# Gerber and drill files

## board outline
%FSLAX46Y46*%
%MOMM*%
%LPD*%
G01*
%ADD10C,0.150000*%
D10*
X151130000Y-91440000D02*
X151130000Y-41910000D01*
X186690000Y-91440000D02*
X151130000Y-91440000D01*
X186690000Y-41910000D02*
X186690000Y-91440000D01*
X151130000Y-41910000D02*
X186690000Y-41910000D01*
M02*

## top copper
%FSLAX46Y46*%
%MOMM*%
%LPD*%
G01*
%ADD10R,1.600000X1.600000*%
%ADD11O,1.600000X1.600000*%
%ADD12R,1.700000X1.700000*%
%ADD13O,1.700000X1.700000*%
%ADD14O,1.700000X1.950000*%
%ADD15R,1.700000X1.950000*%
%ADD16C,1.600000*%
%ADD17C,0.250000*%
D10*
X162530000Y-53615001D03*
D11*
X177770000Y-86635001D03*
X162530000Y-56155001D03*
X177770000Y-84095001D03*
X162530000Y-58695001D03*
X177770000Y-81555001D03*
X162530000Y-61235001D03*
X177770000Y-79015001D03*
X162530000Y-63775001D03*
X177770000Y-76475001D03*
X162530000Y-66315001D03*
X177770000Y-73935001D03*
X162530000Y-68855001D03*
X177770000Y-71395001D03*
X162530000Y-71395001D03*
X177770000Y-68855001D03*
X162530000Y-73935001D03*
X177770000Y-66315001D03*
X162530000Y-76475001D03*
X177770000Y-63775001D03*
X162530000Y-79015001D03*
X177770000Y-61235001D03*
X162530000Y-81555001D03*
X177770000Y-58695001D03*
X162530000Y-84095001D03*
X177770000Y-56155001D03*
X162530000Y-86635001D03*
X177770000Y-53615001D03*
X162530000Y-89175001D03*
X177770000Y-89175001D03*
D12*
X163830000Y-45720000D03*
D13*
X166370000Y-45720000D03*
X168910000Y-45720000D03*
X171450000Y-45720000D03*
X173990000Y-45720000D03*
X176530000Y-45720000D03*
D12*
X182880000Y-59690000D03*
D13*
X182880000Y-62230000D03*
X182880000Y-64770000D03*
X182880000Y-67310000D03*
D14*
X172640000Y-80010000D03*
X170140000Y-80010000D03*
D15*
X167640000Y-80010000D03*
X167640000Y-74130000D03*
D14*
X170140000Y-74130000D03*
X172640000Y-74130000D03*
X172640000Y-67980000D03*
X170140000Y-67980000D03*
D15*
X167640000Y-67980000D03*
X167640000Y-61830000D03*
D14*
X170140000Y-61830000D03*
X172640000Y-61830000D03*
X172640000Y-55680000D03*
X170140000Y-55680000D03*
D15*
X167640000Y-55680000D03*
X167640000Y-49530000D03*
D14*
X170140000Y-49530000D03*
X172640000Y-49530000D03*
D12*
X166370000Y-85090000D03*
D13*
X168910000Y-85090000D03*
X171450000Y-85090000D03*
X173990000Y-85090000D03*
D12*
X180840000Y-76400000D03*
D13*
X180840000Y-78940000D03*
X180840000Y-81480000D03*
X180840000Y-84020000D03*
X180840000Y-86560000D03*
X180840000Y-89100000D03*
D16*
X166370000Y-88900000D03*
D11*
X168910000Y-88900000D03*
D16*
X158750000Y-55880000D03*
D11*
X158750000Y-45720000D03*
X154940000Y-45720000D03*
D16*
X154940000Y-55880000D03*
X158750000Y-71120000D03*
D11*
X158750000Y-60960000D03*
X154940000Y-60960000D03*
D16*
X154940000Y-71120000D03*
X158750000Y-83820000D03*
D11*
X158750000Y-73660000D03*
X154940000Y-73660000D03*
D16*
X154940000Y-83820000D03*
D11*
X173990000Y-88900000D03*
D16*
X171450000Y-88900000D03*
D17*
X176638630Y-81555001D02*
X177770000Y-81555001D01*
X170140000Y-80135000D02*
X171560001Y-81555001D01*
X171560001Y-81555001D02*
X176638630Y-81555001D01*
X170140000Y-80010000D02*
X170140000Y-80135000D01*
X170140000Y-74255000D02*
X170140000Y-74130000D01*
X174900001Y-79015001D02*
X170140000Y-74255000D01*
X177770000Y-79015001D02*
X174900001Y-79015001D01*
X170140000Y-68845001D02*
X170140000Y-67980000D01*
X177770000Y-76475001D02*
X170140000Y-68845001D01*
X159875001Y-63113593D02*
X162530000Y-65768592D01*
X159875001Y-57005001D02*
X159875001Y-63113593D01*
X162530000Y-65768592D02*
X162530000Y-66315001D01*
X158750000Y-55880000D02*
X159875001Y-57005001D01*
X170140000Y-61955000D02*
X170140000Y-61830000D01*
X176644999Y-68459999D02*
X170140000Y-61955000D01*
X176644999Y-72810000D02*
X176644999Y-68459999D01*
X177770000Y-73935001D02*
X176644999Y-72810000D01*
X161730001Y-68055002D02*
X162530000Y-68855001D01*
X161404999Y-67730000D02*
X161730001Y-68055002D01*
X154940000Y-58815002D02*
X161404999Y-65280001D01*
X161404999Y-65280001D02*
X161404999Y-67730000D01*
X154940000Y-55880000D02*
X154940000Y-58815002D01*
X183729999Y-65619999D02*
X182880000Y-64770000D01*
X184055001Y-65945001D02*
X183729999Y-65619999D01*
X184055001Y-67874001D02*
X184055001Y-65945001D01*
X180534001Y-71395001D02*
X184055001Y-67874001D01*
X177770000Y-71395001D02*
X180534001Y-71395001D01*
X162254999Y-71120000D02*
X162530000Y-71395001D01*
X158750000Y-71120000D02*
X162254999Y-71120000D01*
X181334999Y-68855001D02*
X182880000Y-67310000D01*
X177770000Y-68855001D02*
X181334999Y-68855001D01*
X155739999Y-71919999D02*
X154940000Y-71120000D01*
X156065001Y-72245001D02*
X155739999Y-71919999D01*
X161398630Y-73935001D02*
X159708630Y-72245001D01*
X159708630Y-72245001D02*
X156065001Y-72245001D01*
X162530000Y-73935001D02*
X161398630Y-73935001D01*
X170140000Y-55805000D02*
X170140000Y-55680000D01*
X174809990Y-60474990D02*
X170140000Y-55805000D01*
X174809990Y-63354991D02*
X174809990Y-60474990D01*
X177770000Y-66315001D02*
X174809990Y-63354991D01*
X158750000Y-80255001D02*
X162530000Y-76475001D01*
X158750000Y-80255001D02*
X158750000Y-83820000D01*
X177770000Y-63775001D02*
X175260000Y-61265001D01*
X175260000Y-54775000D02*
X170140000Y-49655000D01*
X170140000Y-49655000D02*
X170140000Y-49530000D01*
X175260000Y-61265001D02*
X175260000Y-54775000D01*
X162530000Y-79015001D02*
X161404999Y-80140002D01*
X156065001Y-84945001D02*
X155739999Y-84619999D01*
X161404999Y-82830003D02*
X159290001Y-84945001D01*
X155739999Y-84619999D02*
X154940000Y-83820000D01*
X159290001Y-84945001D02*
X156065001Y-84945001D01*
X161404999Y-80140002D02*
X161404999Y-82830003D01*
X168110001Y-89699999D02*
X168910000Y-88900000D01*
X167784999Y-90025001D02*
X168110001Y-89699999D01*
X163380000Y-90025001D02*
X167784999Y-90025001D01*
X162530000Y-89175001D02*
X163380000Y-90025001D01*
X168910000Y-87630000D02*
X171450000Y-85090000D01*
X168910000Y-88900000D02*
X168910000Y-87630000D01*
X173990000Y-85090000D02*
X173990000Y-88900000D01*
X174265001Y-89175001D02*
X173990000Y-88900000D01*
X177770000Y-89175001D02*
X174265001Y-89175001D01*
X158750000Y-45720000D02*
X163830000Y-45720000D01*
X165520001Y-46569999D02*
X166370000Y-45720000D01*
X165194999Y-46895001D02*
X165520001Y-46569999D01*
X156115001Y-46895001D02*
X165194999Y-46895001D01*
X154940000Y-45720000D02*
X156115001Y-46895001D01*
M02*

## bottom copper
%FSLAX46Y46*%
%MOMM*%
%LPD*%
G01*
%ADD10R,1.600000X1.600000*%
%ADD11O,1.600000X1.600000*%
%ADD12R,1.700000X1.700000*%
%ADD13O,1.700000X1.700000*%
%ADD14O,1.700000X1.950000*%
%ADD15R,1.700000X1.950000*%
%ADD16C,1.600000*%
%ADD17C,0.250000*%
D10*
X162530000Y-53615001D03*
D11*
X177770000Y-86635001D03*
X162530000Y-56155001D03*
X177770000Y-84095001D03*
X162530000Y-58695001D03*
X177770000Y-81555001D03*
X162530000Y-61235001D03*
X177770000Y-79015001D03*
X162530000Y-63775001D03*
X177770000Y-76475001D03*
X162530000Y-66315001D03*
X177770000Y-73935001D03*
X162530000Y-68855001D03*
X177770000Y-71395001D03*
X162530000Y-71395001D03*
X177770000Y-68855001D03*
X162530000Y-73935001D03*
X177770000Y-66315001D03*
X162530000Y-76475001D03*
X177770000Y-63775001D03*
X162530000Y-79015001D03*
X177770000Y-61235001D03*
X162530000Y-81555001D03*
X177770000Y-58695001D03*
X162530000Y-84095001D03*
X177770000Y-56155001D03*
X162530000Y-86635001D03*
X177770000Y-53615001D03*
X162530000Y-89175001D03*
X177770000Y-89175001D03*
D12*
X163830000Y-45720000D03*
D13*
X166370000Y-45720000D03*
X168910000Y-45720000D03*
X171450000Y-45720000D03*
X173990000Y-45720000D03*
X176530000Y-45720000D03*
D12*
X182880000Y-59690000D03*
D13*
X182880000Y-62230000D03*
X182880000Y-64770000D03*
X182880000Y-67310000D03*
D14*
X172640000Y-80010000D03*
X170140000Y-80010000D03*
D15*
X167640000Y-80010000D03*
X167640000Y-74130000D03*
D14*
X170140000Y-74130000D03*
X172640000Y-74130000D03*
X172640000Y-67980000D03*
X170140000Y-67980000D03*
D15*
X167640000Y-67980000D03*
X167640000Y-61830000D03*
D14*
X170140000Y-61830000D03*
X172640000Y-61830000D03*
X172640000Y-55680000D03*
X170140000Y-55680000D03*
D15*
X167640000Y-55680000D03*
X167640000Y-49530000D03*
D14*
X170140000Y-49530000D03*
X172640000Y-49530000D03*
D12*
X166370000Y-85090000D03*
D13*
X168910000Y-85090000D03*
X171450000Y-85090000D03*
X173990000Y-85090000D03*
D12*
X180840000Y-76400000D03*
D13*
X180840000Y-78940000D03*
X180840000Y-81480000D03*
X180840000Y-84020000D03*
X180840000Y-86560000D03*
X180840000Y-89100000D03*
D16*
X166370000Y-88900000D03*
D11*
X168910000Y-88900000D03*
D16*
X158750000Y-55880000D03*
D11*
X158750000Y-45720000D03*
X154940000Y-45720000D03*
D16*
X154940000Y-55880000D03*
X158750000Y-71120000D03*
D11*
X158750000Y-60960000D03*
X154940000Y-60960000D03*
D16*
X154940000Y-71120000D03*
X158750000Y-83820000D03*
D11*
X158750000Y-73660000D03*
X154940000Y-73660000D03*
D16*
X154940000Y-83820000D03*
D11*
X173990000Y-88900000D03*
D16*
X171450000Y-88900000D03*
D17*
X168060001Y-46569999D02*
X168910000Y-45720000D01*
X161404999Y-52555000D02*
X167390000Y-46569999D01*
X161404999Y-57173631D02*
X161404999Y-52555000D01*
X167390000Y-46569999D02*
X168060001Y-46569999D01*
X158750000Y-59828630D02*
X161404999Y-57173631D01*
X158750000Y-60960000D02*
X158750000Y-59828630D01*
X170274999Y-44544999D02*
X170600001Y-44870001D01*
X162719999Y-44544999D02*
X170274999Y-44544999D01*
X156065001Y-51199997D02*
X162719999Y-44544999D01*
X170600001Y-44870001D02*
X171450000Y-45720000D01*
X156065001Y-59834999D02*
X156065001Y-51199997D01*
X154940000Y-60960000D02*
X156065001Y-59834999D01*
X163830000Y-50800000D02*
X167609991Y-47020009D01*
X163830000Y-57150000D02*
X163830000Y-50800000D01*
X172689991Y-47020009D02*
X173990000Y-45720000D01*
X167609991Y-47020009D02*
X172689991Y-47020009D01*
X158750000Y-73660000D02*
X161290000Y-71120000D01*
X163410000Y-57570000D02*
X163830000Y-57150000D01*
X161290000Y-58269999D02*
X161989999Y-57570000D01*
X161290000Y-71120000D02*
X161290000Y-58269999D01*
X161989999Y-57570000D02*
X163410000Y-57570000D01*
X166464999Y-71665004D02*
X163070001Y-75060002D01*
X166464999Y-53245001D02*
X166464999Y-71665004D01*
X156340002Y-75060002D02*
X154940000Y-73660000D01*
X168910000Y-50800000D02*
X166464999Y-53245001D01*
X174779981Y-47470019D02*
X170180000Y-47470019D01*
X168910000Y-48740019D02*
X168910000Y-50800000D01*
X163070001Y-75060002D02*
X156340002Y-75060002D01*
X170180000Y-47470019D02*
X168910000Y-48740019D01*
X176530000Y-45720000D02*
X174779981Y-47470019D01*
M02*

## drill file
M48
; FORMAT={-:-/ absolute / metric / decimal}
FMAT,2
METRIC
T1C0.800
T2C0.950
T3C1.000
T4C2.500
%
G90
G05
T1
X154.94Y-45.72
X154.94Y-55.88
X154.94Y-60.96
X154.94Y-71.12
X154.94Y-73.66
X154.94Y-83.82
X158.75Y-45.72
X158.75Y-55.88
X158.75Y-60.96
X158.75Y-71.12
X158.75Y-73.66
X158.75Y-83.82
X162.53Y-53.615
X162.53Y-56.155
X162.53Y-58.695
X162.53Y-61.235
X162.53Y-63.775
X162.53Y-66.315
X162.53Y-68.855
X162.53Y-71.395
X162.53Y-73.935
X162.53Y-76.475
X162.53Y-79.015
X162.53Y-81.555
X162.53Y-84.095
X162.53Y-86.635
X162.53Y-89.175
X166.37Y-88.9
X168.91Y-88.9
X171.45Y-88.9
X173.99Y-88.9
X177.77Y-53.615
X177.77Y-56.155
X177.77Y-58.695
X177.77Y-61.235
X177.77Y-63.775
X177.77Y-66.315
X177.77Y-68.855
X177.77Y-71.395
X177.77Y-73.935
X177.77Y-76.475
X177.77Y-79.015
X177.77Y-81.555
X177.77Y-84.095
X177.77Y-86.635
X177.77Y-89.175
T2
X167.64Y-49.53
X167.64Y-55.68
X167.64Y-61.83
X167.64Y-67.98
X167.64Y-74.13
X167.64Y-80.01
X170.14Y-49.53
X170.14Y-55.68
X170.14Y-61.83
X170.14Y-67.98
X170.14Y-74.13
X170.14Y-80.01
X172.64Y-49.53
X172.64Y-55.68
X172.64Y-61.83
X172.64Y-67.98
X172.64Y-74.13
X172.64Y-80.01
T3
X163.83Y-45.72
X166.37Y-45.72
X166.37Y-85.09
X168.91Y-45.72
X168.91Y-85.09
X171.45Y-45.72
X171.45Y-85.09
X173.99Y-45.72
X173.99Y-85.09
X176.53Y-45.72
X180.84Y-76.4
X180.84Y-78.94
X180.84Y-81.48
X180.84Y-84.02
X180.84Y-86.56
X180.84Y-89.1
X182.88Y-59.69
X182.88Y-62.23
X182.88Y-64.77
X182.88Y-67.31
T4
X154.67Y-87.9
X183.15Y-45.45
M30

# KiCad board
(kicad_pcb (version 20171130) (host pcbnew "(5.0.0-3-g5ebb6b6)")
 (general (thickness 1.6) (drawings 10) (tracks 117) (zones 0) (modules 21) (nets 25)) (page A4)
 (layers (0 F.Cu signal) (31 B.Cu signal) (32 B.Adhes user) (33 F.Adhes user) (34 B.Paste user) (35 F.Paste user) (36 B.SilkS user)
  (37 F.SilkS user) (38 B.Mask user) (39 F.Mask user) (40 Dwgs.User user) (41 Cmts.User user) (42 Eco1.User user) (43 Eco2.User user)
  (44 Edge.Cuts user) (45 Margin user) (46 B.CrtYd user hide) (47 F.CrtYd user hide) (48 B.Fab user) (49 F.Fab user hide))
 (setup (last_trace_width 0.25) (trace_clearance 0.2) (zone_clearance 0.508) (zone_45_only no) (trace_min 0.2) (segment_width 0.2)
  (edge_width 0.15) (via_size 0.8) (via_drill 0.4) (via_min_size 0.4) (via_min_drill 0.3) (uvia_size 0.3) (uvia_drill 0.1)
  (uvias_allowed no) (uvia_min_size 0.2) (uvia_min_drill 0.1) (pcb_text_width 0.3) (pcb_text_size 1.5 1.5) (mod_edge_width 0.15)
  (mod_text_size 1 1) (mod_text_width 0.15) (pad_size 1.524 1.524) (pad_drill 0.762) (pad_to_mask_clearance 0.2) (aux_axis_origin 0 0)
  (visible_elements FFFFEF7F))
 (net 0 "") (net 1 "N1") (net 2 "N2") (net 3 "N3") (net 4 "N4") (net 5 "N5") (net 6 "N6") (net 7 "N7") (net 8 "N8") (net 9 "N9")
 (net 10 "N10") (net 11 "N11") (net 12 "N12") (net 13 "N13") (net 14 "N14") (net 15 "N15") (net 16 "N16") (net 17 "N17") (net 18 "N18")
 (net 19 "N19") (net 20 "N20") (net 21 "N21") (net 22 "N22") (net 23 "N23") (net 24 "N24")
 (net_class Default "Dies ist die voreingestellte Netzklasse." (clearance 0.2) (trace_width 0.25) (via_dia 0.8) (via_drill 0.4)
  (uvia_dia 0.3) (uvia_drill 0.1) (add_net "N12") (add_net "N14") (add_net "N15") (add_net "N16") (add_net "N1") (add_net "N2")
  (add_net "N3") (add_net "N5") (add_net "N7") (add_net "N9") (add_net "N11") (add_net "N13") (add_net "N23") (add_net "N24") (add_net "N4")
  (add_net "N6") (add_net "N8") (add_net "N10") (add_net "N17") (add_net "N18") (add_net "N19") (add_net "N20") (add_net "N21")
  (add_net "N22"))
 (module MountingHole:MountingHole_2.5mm (layer F.Cu) (at 154.67 87.9)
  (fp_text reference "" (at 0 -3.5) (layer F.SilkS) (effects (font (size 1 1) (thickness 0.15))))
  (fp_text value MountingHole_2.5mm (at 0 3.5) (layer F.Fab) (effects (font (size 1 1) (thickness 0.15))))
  (pad 1 np_thru_hole circle (at 0 0) (size 2.5 2.5) (drill 2.5) (layers *.Cu *.Mask)))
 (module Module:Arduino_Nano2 (layer F.Cu) (at 162.53 53.615001)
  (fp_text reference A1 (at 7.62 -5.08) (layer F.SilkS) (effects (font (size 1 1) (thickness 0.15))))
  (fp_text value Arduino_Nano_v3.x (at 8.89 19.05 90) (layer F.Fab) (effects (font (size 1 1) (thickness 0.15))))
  (pad 1 thru_hole rect (at 0 0) (size 1.6 1.6) (drill 0.8) (layers *.Cu *.Mask))
  (pad 17 thru_hole oval (at 15.24 33.02) (size 1.6 1.6) (drill 0.8) (layers *.Cu *.Mask))
  (pad 2 thru_hole oval (at 0 2.54) (size 1.6 1.6) (drill 0.8) (layers *.Cu *.Mask))
  (pad 18 thru_hole oval (at 15.24 30.48) (size 1.6 1.6) (drill 0.8) (layers *.Cu *.Mask))
  (pad 3 thru_hole oval (at 0 5.08) (size 1.6 1.6) (drill 0.8) (layers *.Cu *.Mask))
  (pad 19 thru_hole oval (at 15.24 27.94) (size 1.6 1.6) (drill 0.8) (layers *.Cu *.Mask) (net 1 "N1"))
  (pad 4 thru_hole oval (at 0 7.62) (size 1.6 1.6) (drill 0.8) (layers *.Cu *.Mask))
  (pad 20 thru_hole oval (at 15.24 25.4) (size 1.6 1.6) (drill 0.8) (layers *.Cu *.Mask) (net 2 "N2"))
  (pad 5 thru_hole oval (at 0 10.16) (size 1.6 1.6) (drill 0.8) (layers *.Cu *.Mask))
  (pad 21 thru_hole oval (at 15.24 22.86) (size 1.6 1.6) (drill 0.8) (layers *.Cu *.Mask) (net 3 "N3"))
  (pad 6 thru_hole oval (at 0 12.7) (size 1.6 1.6) (drill 0.8) (layers *.Cu *.Mask) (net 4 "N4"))
  (pad 22 thru_hole oval (at 15.24 20.32) (size 1.6 1.6) (drill 0.8) (layers *.Cu *.Mask) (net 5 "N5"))
  (pad 7 thru_hole oval (at 0 15.24) (size 1.6 1.6) (drill 0.8) (layers *.Cu *.Mask) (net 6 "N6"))
  (pad 23 thru_hole oval (at 15.24 17.78) (size 1.6 1.6) (drill 0.8) (layers *.Cu *.Mask) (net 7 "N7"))
  (pad 8 thru_hole oval (at 0 17.78) (size 1.6 1.6) (drill 0.8) (layers *.Cu *.Mask) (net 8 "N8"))
  (pad 24 thru_hole oval (at 15.24 15.24) (size 1.6 1.6) (drill 0.8) (layers *.Cu *.Mask) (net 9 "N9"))
  (pad 9 thru_hole oval (at 0 20.32) (size 1.6 1.6) (drill 0.8) (layers *.Cu *.Mask) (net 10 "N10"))
  (pad 25 thru_hole oval (at 15.24 12.7) (size 1.6 1.6) (drill 0.8) (layers *.Cu *.Mask) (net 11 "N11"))
  (pad 10 thru_hole oval (at 0 22.86) (size 1.6 1.6) (drill 0.8) (layers *.Cu *.Mask) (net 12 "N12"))
  (pad 26 thru_hole oval (at 15.24 10.16) (size 1.6 1.6) (drill 0.8) (layers *.Cu *.Mask) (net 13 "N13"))
  (pad 11 thru_hole oval (at 0 25.4) (size 1.6 1.6) (drill 0.8) (layers *.Cu *.Mask) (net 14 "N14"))
  (pad 27 thru_hole oval (at 15.24 7.62) (size 1.6 1.6) (drill 0.8) (layers *.Cu *.Mask))
  (pad 12 thru_hole oval (at 0 27.94) (size 1.6 1.6) (drill 0.8) (layers *.Cu *.Mask))
  (pad 28 thru_hole oval (at 15.24 5.08) (size 1.6 1.6) (drill 0.8) (layers *.Cu *.Mask))
  (pad 13 thru_hole oval (at 0 30.48) (size 1.6 1.6) (drill 0.8) (layers *.Cu *.Mask))
  (pad 29 thru_hole oval (at 15.24 2.54) (size 1.6 1.6) (drill 0.8) (layers *.Cu *.Mask))
  (pad 14 thru_hole oval (at 0 33.02) (size 1.6 1.6) (drill 0.8) (layers *.Cu *.Mask))
  (pad 30 thru_hole oval (at 15.24 0) (size 1.6 1.6) (drill 0.8) (layers *.Cu *.Mask))
  (pad 15 thru_hole oval (at 0 35.56) (size 1.6 1.6) (drill 0.8) (layers *.Cu *.Mask) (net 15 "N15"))
  (pad 16 thru_hole oval (at 15.24 35.56) (size 1.6 1.6) (drill 0.8) (layers *.Cu *.Mask) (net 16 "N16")))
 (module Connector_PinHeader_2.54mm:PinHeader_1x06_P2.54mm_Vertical (layer F.Cu) (at 163.83 45.72 90)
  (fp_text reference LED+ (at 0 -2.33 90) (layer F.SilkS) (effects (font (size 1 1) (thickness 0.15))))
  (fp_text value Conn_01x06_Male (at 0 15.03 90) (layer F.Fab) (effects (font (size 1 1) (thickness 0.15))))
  (pad 1 thru_hole rect (at 0 0 90) (size 1.7 1.7) (drill 1) (layers *.Cu *.Mask) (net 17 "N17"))
  (pad 2 thru_hole oval (at 0 2.54 90) (size 1.7 1.7) (drill 1) (layers *.Cu *.Mask) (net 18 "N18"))
  (pad 3 thru_hole oval (at 0 5.08 90) (size 1.7 1.7) (drill 1) (layers *.Cu *.Mask) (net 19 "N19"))
  (pad 4 thru_hole oval (at 0 7.62 90) (size 1.7 1.7) (drill 1) (layers *.Cu *.Mask) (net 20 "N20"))
  (pad 5 thru_hole oval (at 0 10.16 90) (size 1.7 1.7) (drill 1) (layers *.Cu *.Mask) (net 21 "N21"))
  (pad 6 thru_hole oval (at 0 12.7 90) (size 1.7 1.7) (drill 1) (layers *.Cu *.Mask) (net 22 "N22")))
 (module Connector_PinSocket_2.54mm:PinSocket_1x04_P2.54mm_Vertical (layer F.Cu) (at 182.88 59.69)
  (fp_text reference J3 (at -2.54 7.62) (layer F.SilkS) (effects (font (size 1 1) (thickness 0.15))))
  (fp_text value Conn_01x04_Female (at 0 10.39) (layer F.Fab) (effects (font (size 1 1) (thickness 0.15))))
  (pad 1 thru_hole rect (at 0 0) (size 1.7 1.7) (drill 1) (layers *.Cu *.Mask))
  (pad 2 thru_hole oval (at 0 2.54) (size 1.7 1.7) (drill 1) (layers *.Cu *.Mask))
  (pad 3 thru_hole oval (at 0 5.08) (size 1.7 1.7) (drill 1) (layers *.Cu *.Mask) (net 7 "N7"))
  (pad 4 thru_hole oval (at 0 7.62) (size 1.7 1.7) (drill 1) (layers *.Cu *.Mask) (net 9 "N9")))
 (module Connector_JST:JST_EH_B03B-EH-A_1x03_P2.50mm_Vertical (layer F.Cu) (at 167.64 80.01)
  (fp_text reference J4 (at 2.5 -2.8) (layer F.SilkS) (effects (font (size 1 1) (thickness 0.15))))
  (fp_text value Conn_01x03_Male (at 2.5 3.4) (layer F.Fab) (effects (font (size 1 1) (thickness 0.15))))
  (pad 3 thru_hole oval (at 5 0) (size 1.7 1.95) (drill 0.95) (layers *.Cu *.Mask))
  (pad 2 thru_hole oval (at 2.5 0) (size 1.7 1.95) (drill 0.95) (layers *.Cu *.Mask) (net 1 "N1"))
  (pad 1 thru_hole rect (at 0 0) (size 1.7 1.95) (drill 0.95) (layers *.Cu *.Mask)))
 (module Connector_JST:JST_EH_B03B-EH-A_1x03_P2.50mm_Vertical (layer F.Cu) (at 167.64 74.13)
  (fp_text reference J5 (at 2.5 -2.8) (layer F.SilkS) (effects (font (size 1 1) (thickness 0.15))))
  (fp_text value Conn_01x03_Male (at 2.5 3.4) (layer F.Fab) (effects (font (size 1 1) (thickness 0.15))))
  (pad 1 thru_hole rect (at 0 0) (size 1.7 1.95) (drill 0.95) (layers *.Cu *.Mask))
  (pad 2 thru_hole oval (at 2.5 0) (size 1.7 1.95) (drill 0.95) (layers *.Cu *.Mask) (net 2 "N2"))
  (pad 3 thru_hole oval (at 5 0) (size 1.7 1.95) (drill 0.95) (layers *.Cu *.Mask)))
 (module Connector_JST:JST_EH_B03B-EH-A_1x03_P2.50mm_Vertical (layer F.Cu) (at 167.64 67.98)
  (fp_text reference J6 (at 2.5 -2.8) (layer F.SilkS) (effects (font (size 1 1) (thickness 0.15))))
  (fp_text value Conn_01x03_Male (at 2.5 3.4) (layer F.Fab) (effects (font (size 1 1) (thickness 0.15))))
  (pad 3 thru_hole oval (at 5 0) (size 1.7 1.95) (drill 0.95) (layers *.Cu *.Mask))
  (pad 2 thru_hole oval (at 2.5 0) (size 1.7 1.95) (drill 0.95) (layers *.Cu *.Mask) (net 3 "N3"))
  (pad 1 thru_hole rect (at 0 0) (size 1.7 1.95) (drill 0.95) (layers *.Cu *.Mask)))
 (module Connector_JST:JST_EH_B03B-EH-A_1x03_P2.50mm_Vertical (layer F.Cu) (at 167.64 61.83)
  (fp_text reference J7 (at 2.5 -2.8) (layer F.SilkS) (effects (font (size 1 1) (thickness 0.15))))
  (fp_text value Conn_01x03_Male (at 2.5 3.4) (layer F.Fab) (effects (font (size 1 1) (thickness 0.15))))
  (pad 1 thru_hole rect (at 0 0) (size 1.7 1.95) (drill 0.95) (layers *.Cu *.Mask))
  (pad 2 thru_hole oval (at 2.5 0) (size 1.7 1.95) (drill 0.95) (layers *.Cu *.Mask) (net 5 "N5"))
  (pad 3 thru_hole oval (at 5 0) (size 1.7 1.95) (drill 0.95) (layers *.Cu *.Mask)))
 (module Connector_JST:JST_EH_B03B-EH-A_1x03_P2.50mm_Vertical (layer F.Cu) (at 167.64 55.68)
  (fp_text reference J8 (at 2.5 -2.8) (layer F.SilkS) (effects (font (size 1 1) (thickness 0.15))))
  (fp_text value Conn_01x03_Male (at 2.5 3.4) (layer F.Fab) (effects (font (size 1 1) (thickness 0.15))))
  (pad 3 thru_hole oval (at 5 0) (size 1.7 1.95) (drill 0.95) (layers *.Cu *.Mask))
  (pad 2 thru_hole oval (at 2.5 0) (size 1.7 1.95) (drill 0.95) (layers *.Cu *.Mask) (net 11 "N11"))
  (pad 1 thru_hole rect (at 0 0) (size 1.7 1.95) (drill 0.95) (layers *.Cu *.Mask)))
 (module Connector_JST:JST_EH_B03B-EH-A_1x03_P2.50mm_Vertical (layer F.Cu) (at 167.64 49.53)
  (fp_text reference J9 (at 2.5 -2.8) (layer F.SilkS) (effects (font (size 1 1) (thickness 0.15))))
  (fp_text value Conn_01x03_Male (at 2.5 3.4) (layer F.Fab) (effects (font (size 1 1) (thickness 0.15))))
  (pad 1 thru_hole rect (at 0 0) (size 1.7 1.95) (drill 0.95) (layers *.Cu *.Mask))
  (pad 2 thru_hole oval (at 2.5 0) (size 1.7 1.95) (drill 0.95) (layers *.Cu *.Mask) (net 13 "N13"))
  (pad 3 thru_hole oval (at 5 0) (size 1.7 1.95) (drill 0.95) (layers *.Cu *.Mask)))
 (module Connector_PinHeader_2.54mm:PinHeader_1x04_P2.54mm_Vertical (layer F.Cu) (at 166.37 85.09 90)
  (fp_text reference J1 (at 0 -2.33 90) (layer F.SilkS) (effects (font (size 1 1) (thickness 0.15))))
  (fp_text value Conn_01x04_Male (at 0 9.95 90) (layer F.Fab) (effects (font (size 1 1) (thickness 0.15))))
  (pad 1 thru_hole rect (at 0 0 90) (size 1.7 1.7) (drill 1) (layers *.Cu *.Mask))
  (pad 2 thru_hole oval (at 0 2.54 90) (size 1.7 1.7) (drill 1) (layers *.Cu *.Mask))
  (pad 3 thru_hole oval (at 0 5.08 90) (size 1.7 1.7) (drill 1) (layers *.Cu *.Mask) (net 15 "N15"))
  (pad 4 thru_hole oval (at 0 7.62 90) (size 1.7 1.7) (drill 1) (layers *.Cu *.Mask) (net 16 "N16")))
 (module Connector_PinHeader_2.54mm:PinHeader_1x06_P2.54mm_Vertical (layer F.Cu) (at 180.84 76.4)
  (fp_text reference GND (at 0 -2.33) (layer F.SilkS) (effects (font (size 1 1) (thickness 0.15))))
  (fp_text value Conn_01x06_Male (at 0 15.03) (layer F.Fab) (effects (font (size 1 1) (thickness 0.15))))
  (pad 1 thru_hole rect (at 0 0) (size 1.7 1.7) (drill 1) (layers *.Cu *.Mask))
  (pad 2 thru_hole oval (at 0 2.54) (size 1.7 1.7) (drill 1) (layers *.Cu *.Mask))
  (pad 3 thru_hole oval (at 0 5.08) (size 1.7 1.7) (drill 1) (layers *.Cu *.Mask))
  (pad 4 thru_hole oval (at 0 7.62) (size 1.7 1.7) (drill 1) (layers *.Cu *.Mask))
  (pad 5 thru_hole oval (at 0 10.16) (size 1.7 1.7) (drill 1) (layers *.Cu *.Mask))
  (pad 6 thru_hole oval (at 0 12.7) (size 1.7 1.7) (drill 1) (layers *.Cu *.Mask)))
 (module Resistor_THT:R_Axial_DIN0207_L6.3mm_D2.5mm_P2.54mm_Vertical (layer F.Cu) (at 166.37 88.9)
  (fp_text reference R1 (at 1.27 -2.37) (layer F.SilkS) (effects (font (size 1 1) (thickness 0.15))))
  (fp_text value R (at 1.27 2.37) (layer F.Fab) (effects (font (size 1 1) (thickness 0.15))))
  (pad 1 thru_hole circle (at 0 0) (size 1.6 1.6) (drill 0.8) (layers *.Cu *.Mask))
  (pad 2 thru_hole oval (at 2.54 0) (size 1.6 1.6) (drill 0.8) (layers *.Cu *.Mask) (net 15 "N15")))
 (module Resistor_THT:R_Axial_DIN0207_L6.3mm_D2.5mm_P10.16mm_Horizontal (layer F.Cu) (at 158.75 55.88 90)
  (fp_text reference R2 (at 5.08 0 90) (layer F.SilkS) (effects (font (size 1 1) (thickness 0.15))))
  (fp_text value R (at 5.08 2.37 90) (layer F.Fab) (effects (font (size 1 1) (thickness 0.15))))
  (pad 1 thru_hole circle (at 0 0 90) (size 1.6 1.6) (drill 0.8) (layers *.Cu *.Mask) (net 4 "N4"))
  (pad 2 thru_hole oval (at 10.16 0 90) (size 1.6 1.6) (drill 0.8) (layers *.Cu *.Mask) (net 17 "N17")))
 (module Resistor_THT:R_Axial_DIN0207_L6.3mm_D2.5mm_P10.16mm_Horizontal (layer F.Cu) (at 154.94 55.88 90)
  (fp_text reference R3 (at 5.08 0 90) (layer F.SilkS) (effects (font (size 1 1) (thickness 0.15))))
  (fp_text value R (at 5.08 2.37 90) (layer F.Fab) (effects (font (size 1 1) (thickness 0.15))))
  (pad 2 thru_hole oval (at 10.16 0 90) (size 1.6 1.6) (drill 0.8) (layers *.Cu *.Mask) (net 18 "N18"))
  (pad 1 thru_hole circle (at 0 0 90) (size 1.6 1.6) (drill 0.8) (layers *.Cu *.Mask) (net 6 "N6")))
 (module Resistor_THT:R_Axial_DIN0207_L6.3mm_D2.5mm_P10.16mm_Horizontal (layer F.Cu) (at 158.75 71.12 90)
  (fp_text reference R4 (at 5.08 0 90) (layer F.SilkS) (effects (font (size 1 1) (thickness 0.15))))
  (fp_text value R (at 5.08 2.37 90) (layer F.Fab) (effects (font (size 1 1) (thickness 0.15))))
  (pad 1 thru_hole circle (at 0 0 90) (size 1.6 1.6) (drill 0.8) (layers *.Cu *.Mask) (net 8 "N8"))
  (pad 2 thru_hole oval (at 10.16 0 90) (size 1.6 1.6) (drill 0.8) (layers *.Cu *.Mask) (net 19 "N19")))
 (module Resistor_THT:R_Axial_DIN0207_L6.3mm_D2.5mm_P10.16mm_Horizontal (layer F.Cu) (at 154.94 71.12 90)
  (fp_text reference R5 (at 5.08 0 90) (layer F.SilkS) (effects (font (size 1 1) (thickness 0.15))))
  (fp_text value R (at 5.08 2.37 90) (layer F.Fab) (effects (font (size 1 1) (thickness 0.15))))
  (pad 2 thru_hole oval (at 10.16 0 90) (size 1.6 1.6) (drill 0.8) (layers *.Cu *.Mask) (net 20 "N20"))
  (pad 1 thru_hole circle (at 0 0 90) (size 1.6 1.6) (drill 0.8) (layers *.Cu *.Mask) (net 10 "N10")))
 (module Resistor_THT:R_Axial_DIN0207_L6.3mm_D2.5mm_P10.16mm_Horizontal (layer F.Cu) (at 158.75 83.82 90)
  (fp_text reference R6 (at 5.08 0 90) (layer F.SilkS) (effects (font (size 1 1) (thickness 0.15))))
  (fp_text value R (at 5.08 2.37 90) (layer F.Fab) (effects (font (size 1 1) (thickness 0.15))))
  (pad 1 thru_hole circle (at 0 0 90) (size 1.6 1.6) (drill 0.8) (layers *.Cu *.Mask) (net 12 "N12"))
  (pad 2 thru_hole oval (at 10.16 0 90) (size 1.6 1.6) (drill 0.8) (layers *.Cu *.Mask) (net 21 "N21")))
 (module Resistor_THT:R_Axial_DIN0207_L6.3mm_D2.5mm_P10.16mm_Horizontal (layer F.Cu) (at 154.94 83.82 90)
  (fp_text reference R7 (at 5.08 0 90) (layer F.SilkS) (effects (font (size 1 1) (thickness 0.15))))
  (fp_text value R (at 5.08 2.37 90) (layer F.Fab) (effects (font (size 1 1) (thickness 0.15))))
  (pad 2 thru_hole oval (at 10.16 0 90) (size 1.6 1.6) (drill 0.8) (layers *.Cu *.Mask) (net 22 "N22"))
  (pad 1 thru_hole circle (at 0 0 90) (size 1.6 1.6) (drill 0.8) (layers *.Cu *.Mask) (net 14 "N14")))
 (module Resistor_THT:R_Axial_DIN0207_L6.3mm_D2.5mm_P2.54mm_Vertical (layer F.Cu) (at 171.45 88.9)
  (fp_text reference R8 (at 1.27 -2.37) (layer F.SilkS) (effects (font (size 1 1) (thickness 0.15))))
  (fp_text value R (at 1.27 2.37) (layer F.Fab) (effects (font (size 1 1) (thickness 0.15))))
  (pad 2 thru_hole oval (at 2.54 0) (size 1.6 1.6) (drill 0.8) (layers *.Cu *.Mask) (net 16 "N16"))
  (pad 1 thru_hole circle (at 0 0) (size 1.6 1.6) (drill 0.8) (layers *.Cu *.Mask)))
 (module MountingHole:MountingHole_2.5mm (layer F.Cu) (at 183.15 45.45)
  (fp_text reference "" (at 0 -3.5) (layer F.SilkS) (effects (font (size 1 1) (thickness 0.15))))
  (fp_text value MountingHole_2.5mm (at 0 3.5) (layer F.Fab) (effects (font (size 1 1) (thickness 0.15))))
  (pad 1 np_thru_hole circle (at 0 0) (size 2.5 2.5) (drill 2.5) (layers *.Cu *.Mask)))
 (gr_line (start 151.13 91.44) (end 151.13 41.91) (layer Edge.Cuts) (width 0.15))
 (gr_line (start 186.69 91.44) (end 151.13 91.44) (layer Edge.Cuts) (width 0.15))
 (gr_line (start 186.69 41.91) (end 186.69 91.44) (layer Edge.Cuts) (width 0.15))
 (gr_line (start 151.13 41.91) (end 186.69 41.91) (layer Edge.Cuts) (width 0.15))
 (segment (start 176.63863 81.555001) (end 177.77 81.555001) (width 0.25) (layer F.Cu) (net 1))
 (segment (start 170.14 80.135) (end 171.560001 81.555001) (width 0.25) (layer F.Cu) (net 1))
 (segment (start 171.560001 81.555001) (end 176.63863 81.555001) (width 0.25) (layer F.Cu) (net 1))
 (segment (start 170.14 80.01) (end 170.14 80.135) (width 0.25) (layer F.Cu) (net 1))
 (segment (start 170.14 74.255) (end 170.14 74.13) (width 0.25) (layer F.Cu) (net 2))
 (segment (start 174.900001 79.015001) (end 170.14 74.255) (width 0.25) (layer F.Cu) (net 2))
 (segment (start 177.77 79.015001) (end 174.900001 79.015001) (width 0.25) (layer F.Cu) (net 2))
 (segment (start 170.14 68.845001) (end 170.14 67.98) (width 0.25) (layer F.Cu) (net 3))
 (segment (start 177.77 76.475001) (end 170.14 68.845001) (width 0.25) (layer F.Cu) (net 3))
 (segment (start 159.875001 63.113593) (end 162.53 65.768592) (width 0.25) (layer F.Cu) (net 4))
 (segment (start 159.875001 57.005001) (end 159.875001 63.113593) (width 0.25) (layer F.Cu) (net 4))
 (segment (start 162.53 65.768592) (end 162.53 66.315001) (width 0.25) (layer F.Cu) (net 4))
 (segment (start 158.75 55.88) (end 159.875001 57.005001) (width 0.25) (layer F.Cu) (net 4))
 (segment (start 170.14 61.955) (end 170.14 61.83) (width 0.25) (layer F.Cu) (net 5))
 (segment (start 176.644999 68.459999) (end 170.14 61.955) (width 0.25) (layer F.Cu) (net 5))
 (segment (start 176.644999 72.81) (end 176.644999 68.459999) (width 0.25) (layer F.Cu) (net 5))
 (segment (start 177.77 73.935001) (end 176.644999 72.81) (width 0.25) (layer F.Cu) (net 5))
 (segment (start 161.730001 68.055002) (end 162.53 68.855001) (width 0.25) (layer F.Cu) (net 6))
 (segment (start 161.404999 67.73) (end 161.730001 68.055002) (width 0.25) (layer F.Cu) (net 6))
 (segment (start 154.94 58.815002) (end 161.404999 65.280001) (width 0.25) (layer F.Cu) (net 6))
 (segment (start 161.404999 65.280001) (end 161.404999 67.73) (width 0.25) (layer F.Cu) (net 6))
 (segment (start 154.94 55.88) (end 154.94 58.815002) (width 0.25) (layer F.Cu) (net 6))
 (segment (start 183.729999 65.619999) (end 182.88 64.77) (width 0.25) (layer F.Cu) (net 7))
 (segment (start 184.055001 65.945001) (end 183.729999 65.619999) (width 0.25) (layer F.Cu) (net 7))
 (segment (start 184.055001 67.874001) (end 184.055001 65.945001) (width 0.25) (layer F.Cu) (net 7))
 (segment (start 180.534001 71.395001) (end 184.055001 67.874001) (width 0.25) (layer F.Cu) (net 7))
 (segment (start 177.77 71.395001) (end 180.534001 71.395001) (width 0.25) (layer F.Cu) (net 7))
 (segment (start 162.254999 71.12) (end 162.53 71.395001) (width 0.25) (layer F.Cu) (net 8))
 (segment (start 158.75 71.12) (end 162.254999 71.12) (width 0.25) (layer F.Cu) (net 8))
 (segment (start 181.334999 68.855001) (end 182.88 67.31) (width 0.25) (layer F.Cu) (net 9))
 (segment (start 177.77 68.855001) (end 181.334999 68.855001) (width 0.25) (layer F.Cu) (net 9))
 (segment (start 155.739999 71.919999) (end 154.94 71.12) (width 0.25) (layer F.Cu) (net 10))
 (segment (start 156.065001 72.245001) (end 155.739999 71.919999) (width 0.25) (layer F.Cu) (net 10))
 (segment (start 161.39863 73.935001) (end 159.70863 72.245001) (width 0.25) (layer F.Cu) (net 10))
 (segment (start 159.70863 72.245001) (end 156.065001 72.245001) (width 0.25) (layer F.Cu) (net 10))
 (segment (start 162.53 73.935001) (end 161.39863 73.935001) (width 0.25) (layer F.Cu) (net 10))
 (segment (start 170.14 55.805) (end 170.14 55.68) (width 0.25) (layer F.Cu) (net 11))
 (segment (start 174.80999 60.47499) (end 170.14 55.805) (width 0.25) (layer F.Cu) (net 11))
 (segment (start 174.80999 63.354991) (end 174.80999 60.47499) (width 0.25) (layer F.Cu) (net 11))
 (segment (start 177.77 66.315001) (end 174.80999 63.354991) (width 0.25) (layer F.Cu) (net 11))
 (segment (start 158.75 80.255001) (end 162.53 76.475001) (width 0.25) (layer F.Cu) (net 12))
 (segment (start 158.75 80.255001) (end 158.75 83.82) (width 0.25) (layer F.Cu) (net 12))
 (segment (start 177.77 63.775001) (end 175.26 61.265001) (width 0.25) (layer F.Cu) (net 13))
 (segment (start 175.26 54.775) (end 170.14 49.655) (width 0.25) (layer F.Cu) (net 13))
 (segment (start 170.14 49.655) (end 170.14 49.53) (width 0.25) (layer F.Cu) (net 13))
 (segment (start 175.26 61.265001) (end 175.26 54.775) (width 0.25) (layer F.Cu) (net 13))
 (segment (start 162.53 79.015001) (end 161.404999 80.140002) (width 0.25) (layer F.Cu) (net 14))
 (segment (start 156.065001 84.945001) (end 155.739999 84.619999) (width 0.25) (layer F.Cu) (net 14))
 (segment (start 161.404999 82.830003) (end 159.290001 84.945001) (width 0.25) (layer F.Cu) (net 14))
 (segment (start 155.739999 84.619999) (end 154.94 83.82) (width 0.25) (layer F.Cu) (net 14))
 (segment (start 159.290001 84.945001) (end 156.065001 84.945001) (width 0.25) (layer F.Cu) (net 14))
 (segment (start 161.404999 80.140002) (end 161.404999 82.830003) (width 0.25) (layer F.Cu) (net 14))
 (segment (start 168.110001 89.699999) (end 168.91 88.9) (width 0.25) (layer F.Cu) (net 15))
 (segment (start 167.784999 90.025001) (end 168.110001 89.699999) (width 0.25) (layer F.Cu) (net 15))
 (segment (start 163.38 90.025001) (end 167.784999 90.025001) (width 0.25) (layer F.Cu) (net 15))
 (segment (start 162.53 89.175001) (end 163.38 90.025001) (width 0.25) (layer F.Cu) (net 15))
 (segment (start 168.91 87.63) (end 171.45 85.09) (width 0.25) (layer F.Cu) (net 15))
 (segment (start 168.91 88.9) (end 168.91 87.63) (width 0.25) (layer F.Cu) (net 15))
 (segment (start 173.99 85.09) (end 173.99 88.9) (width 0.25) (layer F.Cu) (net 16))
 (segment (start 174.265001 89.175001) (end 173.99 88.9) (width 0.25) (layer F.Cu) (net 16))
 (segment (start 177.77 89.175001) (end 174.265001 89.175001) (width 0.25) (layer F.Cu) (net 16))
 (segment (start 158.75 45.72) (end 163.83 45.72) (width 0.25) (layer F.Cu) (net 17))
 (segment (start 165.520001 46.569999) (end 166.37 45.72) (width 0.25) (layer F.Cu) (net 18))
 (segment (start 165.194999 46.895001) (end 165.520001 46.569999) (width 0.25) (layer F.Cu) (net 18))
 (segment (start 156.115001 46.895001) (end 165.194999 46.895001) (width 0.25) (layer F.Cu) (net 18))
 (segment (start 154.94 45.72) (end 156.115001 46.895001) (width 0.25) (layer F.Cu) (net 18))
 (segment (start 168.060001 46.569999) (end 168.91 45.72) (width 0.25) (layer B.Cu) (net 19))
 (segment (start 161.404999 52.555) (end 167.39 46.569999) (width 0.25) (layer B.Cu) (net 19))
 (segment (start 161.404999 57.173631) (end 161.404999 52.555) (width 0.25) (layer B.Cu) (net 19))
 (segment (start 167.39 46.569999) (end 168.060001 46.569999) (width 0.25) (layer B.Cu) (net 19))
 (segment (start 158.75 59.82863) (end 161.404999 57.173631) (width 0.25) (layer B.Cu) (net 19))
 (segment (start 158.75 60.96) (end 158.75 59.82863) (width 0.25) (layer B.Cu) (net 19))
 (segment (start 170.274999 44.544999) (end 170.600001 44.870001) (width 0.25) (layer B.Cu) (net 20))
 (segment (start 162.719999 44.544999) (end 170.274999 44.544999) (width 0.25) (layer B.Cu) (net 20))
 (segment (start 156.065001 51.199997) (end 162.719999 44.544999) (width 0.25) (layer B.Cu) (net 20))
 (segment (start 170.600001 44.870001) (end 171.45 45.72) (width 0.25) (layer B.Cu) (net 20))
 (segment (start 156.065001 59.834999) (end 156.065001 51.199997) (width 0.25) (layer B.Cu) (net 20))
 (segment (start 154.94 60.96) (end 156.065001 59.834999) (width 0.25) (layer B.Cu) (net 20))
 (segment (start 163.83 50.8) (end 167.609991 47.020009) (width 0.25) (layer B.Cu) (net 21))
 (segment (start 163.83 57.15) (end 163.83 50.8) (width 0.25) (layer B.Cu) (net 21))
 (segment (start 172.689991 47.020009) (end 173.99 45.72) (width 0.25) (layer B.Cu) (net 21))
 (segment (start 167.609991 47.020009) (end 172.689991 47.020009) (width 0.25) (layer B.Cu) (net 21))
 (segment (start 158.75 73.66) (end 161.29 71.12) (width 0.25) (layer B.Cu) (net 21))
 (segment (start 163.41 57.57) (end 163.83 57.15) (width 0.25) (layer B.Cu) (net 21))
 (segment (start 161.29 58.269999) (end 161.989999 57.57) (width 0.25) (layer B.Cu) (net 21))
 (segment (start 161.29 71.12) (end 161.29 58.269999) (width 0.25) (layer B.Cu) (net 21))
 (segment (start 161.989999 57.57) (end 163.41 57.57) (width 0.25) (layer B.Cu) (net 21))
 (segment (start 166.464999 71.665004) (end 163.070001 75.060002) (width 0.25) (layer B.Cu) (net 22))
 (segment (start 166.464999 53.245001) (end 166.464999 71.665004) (width 0.25) (layer B.Cu) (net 22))
 (segment (start 156.340002 75.060002) (end 154.94 73.66) (width 0.25) (layer B.Cu) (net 22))
 (segment (start 168.91 50.8) (end 166.464999 53.245001) (width 0.25) (layer B.Cu) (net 22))
 (segment (start 174.779981 47.470019) (end 170.18 47.470019) (width 0.25) (layer B.Cu) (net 22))
 (segment (start 168.91 48.740019) (end 168.91 50.8) (width 0.25) (layer B.Cu) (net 22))
 (segment (start 163.070001 75.060002) (end 156.340002 75.060002) (width 0.25) (layer B.Cu) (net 22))
 (segment (start 170.18 47.470019) (end 168.91 48.740019) (width 0.25) (layer B.Cu) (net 22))
 (segment (start 176.53 45.72) (end 174.779981 47.470019) (width 0.25) (layer B.Cu) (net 22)))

